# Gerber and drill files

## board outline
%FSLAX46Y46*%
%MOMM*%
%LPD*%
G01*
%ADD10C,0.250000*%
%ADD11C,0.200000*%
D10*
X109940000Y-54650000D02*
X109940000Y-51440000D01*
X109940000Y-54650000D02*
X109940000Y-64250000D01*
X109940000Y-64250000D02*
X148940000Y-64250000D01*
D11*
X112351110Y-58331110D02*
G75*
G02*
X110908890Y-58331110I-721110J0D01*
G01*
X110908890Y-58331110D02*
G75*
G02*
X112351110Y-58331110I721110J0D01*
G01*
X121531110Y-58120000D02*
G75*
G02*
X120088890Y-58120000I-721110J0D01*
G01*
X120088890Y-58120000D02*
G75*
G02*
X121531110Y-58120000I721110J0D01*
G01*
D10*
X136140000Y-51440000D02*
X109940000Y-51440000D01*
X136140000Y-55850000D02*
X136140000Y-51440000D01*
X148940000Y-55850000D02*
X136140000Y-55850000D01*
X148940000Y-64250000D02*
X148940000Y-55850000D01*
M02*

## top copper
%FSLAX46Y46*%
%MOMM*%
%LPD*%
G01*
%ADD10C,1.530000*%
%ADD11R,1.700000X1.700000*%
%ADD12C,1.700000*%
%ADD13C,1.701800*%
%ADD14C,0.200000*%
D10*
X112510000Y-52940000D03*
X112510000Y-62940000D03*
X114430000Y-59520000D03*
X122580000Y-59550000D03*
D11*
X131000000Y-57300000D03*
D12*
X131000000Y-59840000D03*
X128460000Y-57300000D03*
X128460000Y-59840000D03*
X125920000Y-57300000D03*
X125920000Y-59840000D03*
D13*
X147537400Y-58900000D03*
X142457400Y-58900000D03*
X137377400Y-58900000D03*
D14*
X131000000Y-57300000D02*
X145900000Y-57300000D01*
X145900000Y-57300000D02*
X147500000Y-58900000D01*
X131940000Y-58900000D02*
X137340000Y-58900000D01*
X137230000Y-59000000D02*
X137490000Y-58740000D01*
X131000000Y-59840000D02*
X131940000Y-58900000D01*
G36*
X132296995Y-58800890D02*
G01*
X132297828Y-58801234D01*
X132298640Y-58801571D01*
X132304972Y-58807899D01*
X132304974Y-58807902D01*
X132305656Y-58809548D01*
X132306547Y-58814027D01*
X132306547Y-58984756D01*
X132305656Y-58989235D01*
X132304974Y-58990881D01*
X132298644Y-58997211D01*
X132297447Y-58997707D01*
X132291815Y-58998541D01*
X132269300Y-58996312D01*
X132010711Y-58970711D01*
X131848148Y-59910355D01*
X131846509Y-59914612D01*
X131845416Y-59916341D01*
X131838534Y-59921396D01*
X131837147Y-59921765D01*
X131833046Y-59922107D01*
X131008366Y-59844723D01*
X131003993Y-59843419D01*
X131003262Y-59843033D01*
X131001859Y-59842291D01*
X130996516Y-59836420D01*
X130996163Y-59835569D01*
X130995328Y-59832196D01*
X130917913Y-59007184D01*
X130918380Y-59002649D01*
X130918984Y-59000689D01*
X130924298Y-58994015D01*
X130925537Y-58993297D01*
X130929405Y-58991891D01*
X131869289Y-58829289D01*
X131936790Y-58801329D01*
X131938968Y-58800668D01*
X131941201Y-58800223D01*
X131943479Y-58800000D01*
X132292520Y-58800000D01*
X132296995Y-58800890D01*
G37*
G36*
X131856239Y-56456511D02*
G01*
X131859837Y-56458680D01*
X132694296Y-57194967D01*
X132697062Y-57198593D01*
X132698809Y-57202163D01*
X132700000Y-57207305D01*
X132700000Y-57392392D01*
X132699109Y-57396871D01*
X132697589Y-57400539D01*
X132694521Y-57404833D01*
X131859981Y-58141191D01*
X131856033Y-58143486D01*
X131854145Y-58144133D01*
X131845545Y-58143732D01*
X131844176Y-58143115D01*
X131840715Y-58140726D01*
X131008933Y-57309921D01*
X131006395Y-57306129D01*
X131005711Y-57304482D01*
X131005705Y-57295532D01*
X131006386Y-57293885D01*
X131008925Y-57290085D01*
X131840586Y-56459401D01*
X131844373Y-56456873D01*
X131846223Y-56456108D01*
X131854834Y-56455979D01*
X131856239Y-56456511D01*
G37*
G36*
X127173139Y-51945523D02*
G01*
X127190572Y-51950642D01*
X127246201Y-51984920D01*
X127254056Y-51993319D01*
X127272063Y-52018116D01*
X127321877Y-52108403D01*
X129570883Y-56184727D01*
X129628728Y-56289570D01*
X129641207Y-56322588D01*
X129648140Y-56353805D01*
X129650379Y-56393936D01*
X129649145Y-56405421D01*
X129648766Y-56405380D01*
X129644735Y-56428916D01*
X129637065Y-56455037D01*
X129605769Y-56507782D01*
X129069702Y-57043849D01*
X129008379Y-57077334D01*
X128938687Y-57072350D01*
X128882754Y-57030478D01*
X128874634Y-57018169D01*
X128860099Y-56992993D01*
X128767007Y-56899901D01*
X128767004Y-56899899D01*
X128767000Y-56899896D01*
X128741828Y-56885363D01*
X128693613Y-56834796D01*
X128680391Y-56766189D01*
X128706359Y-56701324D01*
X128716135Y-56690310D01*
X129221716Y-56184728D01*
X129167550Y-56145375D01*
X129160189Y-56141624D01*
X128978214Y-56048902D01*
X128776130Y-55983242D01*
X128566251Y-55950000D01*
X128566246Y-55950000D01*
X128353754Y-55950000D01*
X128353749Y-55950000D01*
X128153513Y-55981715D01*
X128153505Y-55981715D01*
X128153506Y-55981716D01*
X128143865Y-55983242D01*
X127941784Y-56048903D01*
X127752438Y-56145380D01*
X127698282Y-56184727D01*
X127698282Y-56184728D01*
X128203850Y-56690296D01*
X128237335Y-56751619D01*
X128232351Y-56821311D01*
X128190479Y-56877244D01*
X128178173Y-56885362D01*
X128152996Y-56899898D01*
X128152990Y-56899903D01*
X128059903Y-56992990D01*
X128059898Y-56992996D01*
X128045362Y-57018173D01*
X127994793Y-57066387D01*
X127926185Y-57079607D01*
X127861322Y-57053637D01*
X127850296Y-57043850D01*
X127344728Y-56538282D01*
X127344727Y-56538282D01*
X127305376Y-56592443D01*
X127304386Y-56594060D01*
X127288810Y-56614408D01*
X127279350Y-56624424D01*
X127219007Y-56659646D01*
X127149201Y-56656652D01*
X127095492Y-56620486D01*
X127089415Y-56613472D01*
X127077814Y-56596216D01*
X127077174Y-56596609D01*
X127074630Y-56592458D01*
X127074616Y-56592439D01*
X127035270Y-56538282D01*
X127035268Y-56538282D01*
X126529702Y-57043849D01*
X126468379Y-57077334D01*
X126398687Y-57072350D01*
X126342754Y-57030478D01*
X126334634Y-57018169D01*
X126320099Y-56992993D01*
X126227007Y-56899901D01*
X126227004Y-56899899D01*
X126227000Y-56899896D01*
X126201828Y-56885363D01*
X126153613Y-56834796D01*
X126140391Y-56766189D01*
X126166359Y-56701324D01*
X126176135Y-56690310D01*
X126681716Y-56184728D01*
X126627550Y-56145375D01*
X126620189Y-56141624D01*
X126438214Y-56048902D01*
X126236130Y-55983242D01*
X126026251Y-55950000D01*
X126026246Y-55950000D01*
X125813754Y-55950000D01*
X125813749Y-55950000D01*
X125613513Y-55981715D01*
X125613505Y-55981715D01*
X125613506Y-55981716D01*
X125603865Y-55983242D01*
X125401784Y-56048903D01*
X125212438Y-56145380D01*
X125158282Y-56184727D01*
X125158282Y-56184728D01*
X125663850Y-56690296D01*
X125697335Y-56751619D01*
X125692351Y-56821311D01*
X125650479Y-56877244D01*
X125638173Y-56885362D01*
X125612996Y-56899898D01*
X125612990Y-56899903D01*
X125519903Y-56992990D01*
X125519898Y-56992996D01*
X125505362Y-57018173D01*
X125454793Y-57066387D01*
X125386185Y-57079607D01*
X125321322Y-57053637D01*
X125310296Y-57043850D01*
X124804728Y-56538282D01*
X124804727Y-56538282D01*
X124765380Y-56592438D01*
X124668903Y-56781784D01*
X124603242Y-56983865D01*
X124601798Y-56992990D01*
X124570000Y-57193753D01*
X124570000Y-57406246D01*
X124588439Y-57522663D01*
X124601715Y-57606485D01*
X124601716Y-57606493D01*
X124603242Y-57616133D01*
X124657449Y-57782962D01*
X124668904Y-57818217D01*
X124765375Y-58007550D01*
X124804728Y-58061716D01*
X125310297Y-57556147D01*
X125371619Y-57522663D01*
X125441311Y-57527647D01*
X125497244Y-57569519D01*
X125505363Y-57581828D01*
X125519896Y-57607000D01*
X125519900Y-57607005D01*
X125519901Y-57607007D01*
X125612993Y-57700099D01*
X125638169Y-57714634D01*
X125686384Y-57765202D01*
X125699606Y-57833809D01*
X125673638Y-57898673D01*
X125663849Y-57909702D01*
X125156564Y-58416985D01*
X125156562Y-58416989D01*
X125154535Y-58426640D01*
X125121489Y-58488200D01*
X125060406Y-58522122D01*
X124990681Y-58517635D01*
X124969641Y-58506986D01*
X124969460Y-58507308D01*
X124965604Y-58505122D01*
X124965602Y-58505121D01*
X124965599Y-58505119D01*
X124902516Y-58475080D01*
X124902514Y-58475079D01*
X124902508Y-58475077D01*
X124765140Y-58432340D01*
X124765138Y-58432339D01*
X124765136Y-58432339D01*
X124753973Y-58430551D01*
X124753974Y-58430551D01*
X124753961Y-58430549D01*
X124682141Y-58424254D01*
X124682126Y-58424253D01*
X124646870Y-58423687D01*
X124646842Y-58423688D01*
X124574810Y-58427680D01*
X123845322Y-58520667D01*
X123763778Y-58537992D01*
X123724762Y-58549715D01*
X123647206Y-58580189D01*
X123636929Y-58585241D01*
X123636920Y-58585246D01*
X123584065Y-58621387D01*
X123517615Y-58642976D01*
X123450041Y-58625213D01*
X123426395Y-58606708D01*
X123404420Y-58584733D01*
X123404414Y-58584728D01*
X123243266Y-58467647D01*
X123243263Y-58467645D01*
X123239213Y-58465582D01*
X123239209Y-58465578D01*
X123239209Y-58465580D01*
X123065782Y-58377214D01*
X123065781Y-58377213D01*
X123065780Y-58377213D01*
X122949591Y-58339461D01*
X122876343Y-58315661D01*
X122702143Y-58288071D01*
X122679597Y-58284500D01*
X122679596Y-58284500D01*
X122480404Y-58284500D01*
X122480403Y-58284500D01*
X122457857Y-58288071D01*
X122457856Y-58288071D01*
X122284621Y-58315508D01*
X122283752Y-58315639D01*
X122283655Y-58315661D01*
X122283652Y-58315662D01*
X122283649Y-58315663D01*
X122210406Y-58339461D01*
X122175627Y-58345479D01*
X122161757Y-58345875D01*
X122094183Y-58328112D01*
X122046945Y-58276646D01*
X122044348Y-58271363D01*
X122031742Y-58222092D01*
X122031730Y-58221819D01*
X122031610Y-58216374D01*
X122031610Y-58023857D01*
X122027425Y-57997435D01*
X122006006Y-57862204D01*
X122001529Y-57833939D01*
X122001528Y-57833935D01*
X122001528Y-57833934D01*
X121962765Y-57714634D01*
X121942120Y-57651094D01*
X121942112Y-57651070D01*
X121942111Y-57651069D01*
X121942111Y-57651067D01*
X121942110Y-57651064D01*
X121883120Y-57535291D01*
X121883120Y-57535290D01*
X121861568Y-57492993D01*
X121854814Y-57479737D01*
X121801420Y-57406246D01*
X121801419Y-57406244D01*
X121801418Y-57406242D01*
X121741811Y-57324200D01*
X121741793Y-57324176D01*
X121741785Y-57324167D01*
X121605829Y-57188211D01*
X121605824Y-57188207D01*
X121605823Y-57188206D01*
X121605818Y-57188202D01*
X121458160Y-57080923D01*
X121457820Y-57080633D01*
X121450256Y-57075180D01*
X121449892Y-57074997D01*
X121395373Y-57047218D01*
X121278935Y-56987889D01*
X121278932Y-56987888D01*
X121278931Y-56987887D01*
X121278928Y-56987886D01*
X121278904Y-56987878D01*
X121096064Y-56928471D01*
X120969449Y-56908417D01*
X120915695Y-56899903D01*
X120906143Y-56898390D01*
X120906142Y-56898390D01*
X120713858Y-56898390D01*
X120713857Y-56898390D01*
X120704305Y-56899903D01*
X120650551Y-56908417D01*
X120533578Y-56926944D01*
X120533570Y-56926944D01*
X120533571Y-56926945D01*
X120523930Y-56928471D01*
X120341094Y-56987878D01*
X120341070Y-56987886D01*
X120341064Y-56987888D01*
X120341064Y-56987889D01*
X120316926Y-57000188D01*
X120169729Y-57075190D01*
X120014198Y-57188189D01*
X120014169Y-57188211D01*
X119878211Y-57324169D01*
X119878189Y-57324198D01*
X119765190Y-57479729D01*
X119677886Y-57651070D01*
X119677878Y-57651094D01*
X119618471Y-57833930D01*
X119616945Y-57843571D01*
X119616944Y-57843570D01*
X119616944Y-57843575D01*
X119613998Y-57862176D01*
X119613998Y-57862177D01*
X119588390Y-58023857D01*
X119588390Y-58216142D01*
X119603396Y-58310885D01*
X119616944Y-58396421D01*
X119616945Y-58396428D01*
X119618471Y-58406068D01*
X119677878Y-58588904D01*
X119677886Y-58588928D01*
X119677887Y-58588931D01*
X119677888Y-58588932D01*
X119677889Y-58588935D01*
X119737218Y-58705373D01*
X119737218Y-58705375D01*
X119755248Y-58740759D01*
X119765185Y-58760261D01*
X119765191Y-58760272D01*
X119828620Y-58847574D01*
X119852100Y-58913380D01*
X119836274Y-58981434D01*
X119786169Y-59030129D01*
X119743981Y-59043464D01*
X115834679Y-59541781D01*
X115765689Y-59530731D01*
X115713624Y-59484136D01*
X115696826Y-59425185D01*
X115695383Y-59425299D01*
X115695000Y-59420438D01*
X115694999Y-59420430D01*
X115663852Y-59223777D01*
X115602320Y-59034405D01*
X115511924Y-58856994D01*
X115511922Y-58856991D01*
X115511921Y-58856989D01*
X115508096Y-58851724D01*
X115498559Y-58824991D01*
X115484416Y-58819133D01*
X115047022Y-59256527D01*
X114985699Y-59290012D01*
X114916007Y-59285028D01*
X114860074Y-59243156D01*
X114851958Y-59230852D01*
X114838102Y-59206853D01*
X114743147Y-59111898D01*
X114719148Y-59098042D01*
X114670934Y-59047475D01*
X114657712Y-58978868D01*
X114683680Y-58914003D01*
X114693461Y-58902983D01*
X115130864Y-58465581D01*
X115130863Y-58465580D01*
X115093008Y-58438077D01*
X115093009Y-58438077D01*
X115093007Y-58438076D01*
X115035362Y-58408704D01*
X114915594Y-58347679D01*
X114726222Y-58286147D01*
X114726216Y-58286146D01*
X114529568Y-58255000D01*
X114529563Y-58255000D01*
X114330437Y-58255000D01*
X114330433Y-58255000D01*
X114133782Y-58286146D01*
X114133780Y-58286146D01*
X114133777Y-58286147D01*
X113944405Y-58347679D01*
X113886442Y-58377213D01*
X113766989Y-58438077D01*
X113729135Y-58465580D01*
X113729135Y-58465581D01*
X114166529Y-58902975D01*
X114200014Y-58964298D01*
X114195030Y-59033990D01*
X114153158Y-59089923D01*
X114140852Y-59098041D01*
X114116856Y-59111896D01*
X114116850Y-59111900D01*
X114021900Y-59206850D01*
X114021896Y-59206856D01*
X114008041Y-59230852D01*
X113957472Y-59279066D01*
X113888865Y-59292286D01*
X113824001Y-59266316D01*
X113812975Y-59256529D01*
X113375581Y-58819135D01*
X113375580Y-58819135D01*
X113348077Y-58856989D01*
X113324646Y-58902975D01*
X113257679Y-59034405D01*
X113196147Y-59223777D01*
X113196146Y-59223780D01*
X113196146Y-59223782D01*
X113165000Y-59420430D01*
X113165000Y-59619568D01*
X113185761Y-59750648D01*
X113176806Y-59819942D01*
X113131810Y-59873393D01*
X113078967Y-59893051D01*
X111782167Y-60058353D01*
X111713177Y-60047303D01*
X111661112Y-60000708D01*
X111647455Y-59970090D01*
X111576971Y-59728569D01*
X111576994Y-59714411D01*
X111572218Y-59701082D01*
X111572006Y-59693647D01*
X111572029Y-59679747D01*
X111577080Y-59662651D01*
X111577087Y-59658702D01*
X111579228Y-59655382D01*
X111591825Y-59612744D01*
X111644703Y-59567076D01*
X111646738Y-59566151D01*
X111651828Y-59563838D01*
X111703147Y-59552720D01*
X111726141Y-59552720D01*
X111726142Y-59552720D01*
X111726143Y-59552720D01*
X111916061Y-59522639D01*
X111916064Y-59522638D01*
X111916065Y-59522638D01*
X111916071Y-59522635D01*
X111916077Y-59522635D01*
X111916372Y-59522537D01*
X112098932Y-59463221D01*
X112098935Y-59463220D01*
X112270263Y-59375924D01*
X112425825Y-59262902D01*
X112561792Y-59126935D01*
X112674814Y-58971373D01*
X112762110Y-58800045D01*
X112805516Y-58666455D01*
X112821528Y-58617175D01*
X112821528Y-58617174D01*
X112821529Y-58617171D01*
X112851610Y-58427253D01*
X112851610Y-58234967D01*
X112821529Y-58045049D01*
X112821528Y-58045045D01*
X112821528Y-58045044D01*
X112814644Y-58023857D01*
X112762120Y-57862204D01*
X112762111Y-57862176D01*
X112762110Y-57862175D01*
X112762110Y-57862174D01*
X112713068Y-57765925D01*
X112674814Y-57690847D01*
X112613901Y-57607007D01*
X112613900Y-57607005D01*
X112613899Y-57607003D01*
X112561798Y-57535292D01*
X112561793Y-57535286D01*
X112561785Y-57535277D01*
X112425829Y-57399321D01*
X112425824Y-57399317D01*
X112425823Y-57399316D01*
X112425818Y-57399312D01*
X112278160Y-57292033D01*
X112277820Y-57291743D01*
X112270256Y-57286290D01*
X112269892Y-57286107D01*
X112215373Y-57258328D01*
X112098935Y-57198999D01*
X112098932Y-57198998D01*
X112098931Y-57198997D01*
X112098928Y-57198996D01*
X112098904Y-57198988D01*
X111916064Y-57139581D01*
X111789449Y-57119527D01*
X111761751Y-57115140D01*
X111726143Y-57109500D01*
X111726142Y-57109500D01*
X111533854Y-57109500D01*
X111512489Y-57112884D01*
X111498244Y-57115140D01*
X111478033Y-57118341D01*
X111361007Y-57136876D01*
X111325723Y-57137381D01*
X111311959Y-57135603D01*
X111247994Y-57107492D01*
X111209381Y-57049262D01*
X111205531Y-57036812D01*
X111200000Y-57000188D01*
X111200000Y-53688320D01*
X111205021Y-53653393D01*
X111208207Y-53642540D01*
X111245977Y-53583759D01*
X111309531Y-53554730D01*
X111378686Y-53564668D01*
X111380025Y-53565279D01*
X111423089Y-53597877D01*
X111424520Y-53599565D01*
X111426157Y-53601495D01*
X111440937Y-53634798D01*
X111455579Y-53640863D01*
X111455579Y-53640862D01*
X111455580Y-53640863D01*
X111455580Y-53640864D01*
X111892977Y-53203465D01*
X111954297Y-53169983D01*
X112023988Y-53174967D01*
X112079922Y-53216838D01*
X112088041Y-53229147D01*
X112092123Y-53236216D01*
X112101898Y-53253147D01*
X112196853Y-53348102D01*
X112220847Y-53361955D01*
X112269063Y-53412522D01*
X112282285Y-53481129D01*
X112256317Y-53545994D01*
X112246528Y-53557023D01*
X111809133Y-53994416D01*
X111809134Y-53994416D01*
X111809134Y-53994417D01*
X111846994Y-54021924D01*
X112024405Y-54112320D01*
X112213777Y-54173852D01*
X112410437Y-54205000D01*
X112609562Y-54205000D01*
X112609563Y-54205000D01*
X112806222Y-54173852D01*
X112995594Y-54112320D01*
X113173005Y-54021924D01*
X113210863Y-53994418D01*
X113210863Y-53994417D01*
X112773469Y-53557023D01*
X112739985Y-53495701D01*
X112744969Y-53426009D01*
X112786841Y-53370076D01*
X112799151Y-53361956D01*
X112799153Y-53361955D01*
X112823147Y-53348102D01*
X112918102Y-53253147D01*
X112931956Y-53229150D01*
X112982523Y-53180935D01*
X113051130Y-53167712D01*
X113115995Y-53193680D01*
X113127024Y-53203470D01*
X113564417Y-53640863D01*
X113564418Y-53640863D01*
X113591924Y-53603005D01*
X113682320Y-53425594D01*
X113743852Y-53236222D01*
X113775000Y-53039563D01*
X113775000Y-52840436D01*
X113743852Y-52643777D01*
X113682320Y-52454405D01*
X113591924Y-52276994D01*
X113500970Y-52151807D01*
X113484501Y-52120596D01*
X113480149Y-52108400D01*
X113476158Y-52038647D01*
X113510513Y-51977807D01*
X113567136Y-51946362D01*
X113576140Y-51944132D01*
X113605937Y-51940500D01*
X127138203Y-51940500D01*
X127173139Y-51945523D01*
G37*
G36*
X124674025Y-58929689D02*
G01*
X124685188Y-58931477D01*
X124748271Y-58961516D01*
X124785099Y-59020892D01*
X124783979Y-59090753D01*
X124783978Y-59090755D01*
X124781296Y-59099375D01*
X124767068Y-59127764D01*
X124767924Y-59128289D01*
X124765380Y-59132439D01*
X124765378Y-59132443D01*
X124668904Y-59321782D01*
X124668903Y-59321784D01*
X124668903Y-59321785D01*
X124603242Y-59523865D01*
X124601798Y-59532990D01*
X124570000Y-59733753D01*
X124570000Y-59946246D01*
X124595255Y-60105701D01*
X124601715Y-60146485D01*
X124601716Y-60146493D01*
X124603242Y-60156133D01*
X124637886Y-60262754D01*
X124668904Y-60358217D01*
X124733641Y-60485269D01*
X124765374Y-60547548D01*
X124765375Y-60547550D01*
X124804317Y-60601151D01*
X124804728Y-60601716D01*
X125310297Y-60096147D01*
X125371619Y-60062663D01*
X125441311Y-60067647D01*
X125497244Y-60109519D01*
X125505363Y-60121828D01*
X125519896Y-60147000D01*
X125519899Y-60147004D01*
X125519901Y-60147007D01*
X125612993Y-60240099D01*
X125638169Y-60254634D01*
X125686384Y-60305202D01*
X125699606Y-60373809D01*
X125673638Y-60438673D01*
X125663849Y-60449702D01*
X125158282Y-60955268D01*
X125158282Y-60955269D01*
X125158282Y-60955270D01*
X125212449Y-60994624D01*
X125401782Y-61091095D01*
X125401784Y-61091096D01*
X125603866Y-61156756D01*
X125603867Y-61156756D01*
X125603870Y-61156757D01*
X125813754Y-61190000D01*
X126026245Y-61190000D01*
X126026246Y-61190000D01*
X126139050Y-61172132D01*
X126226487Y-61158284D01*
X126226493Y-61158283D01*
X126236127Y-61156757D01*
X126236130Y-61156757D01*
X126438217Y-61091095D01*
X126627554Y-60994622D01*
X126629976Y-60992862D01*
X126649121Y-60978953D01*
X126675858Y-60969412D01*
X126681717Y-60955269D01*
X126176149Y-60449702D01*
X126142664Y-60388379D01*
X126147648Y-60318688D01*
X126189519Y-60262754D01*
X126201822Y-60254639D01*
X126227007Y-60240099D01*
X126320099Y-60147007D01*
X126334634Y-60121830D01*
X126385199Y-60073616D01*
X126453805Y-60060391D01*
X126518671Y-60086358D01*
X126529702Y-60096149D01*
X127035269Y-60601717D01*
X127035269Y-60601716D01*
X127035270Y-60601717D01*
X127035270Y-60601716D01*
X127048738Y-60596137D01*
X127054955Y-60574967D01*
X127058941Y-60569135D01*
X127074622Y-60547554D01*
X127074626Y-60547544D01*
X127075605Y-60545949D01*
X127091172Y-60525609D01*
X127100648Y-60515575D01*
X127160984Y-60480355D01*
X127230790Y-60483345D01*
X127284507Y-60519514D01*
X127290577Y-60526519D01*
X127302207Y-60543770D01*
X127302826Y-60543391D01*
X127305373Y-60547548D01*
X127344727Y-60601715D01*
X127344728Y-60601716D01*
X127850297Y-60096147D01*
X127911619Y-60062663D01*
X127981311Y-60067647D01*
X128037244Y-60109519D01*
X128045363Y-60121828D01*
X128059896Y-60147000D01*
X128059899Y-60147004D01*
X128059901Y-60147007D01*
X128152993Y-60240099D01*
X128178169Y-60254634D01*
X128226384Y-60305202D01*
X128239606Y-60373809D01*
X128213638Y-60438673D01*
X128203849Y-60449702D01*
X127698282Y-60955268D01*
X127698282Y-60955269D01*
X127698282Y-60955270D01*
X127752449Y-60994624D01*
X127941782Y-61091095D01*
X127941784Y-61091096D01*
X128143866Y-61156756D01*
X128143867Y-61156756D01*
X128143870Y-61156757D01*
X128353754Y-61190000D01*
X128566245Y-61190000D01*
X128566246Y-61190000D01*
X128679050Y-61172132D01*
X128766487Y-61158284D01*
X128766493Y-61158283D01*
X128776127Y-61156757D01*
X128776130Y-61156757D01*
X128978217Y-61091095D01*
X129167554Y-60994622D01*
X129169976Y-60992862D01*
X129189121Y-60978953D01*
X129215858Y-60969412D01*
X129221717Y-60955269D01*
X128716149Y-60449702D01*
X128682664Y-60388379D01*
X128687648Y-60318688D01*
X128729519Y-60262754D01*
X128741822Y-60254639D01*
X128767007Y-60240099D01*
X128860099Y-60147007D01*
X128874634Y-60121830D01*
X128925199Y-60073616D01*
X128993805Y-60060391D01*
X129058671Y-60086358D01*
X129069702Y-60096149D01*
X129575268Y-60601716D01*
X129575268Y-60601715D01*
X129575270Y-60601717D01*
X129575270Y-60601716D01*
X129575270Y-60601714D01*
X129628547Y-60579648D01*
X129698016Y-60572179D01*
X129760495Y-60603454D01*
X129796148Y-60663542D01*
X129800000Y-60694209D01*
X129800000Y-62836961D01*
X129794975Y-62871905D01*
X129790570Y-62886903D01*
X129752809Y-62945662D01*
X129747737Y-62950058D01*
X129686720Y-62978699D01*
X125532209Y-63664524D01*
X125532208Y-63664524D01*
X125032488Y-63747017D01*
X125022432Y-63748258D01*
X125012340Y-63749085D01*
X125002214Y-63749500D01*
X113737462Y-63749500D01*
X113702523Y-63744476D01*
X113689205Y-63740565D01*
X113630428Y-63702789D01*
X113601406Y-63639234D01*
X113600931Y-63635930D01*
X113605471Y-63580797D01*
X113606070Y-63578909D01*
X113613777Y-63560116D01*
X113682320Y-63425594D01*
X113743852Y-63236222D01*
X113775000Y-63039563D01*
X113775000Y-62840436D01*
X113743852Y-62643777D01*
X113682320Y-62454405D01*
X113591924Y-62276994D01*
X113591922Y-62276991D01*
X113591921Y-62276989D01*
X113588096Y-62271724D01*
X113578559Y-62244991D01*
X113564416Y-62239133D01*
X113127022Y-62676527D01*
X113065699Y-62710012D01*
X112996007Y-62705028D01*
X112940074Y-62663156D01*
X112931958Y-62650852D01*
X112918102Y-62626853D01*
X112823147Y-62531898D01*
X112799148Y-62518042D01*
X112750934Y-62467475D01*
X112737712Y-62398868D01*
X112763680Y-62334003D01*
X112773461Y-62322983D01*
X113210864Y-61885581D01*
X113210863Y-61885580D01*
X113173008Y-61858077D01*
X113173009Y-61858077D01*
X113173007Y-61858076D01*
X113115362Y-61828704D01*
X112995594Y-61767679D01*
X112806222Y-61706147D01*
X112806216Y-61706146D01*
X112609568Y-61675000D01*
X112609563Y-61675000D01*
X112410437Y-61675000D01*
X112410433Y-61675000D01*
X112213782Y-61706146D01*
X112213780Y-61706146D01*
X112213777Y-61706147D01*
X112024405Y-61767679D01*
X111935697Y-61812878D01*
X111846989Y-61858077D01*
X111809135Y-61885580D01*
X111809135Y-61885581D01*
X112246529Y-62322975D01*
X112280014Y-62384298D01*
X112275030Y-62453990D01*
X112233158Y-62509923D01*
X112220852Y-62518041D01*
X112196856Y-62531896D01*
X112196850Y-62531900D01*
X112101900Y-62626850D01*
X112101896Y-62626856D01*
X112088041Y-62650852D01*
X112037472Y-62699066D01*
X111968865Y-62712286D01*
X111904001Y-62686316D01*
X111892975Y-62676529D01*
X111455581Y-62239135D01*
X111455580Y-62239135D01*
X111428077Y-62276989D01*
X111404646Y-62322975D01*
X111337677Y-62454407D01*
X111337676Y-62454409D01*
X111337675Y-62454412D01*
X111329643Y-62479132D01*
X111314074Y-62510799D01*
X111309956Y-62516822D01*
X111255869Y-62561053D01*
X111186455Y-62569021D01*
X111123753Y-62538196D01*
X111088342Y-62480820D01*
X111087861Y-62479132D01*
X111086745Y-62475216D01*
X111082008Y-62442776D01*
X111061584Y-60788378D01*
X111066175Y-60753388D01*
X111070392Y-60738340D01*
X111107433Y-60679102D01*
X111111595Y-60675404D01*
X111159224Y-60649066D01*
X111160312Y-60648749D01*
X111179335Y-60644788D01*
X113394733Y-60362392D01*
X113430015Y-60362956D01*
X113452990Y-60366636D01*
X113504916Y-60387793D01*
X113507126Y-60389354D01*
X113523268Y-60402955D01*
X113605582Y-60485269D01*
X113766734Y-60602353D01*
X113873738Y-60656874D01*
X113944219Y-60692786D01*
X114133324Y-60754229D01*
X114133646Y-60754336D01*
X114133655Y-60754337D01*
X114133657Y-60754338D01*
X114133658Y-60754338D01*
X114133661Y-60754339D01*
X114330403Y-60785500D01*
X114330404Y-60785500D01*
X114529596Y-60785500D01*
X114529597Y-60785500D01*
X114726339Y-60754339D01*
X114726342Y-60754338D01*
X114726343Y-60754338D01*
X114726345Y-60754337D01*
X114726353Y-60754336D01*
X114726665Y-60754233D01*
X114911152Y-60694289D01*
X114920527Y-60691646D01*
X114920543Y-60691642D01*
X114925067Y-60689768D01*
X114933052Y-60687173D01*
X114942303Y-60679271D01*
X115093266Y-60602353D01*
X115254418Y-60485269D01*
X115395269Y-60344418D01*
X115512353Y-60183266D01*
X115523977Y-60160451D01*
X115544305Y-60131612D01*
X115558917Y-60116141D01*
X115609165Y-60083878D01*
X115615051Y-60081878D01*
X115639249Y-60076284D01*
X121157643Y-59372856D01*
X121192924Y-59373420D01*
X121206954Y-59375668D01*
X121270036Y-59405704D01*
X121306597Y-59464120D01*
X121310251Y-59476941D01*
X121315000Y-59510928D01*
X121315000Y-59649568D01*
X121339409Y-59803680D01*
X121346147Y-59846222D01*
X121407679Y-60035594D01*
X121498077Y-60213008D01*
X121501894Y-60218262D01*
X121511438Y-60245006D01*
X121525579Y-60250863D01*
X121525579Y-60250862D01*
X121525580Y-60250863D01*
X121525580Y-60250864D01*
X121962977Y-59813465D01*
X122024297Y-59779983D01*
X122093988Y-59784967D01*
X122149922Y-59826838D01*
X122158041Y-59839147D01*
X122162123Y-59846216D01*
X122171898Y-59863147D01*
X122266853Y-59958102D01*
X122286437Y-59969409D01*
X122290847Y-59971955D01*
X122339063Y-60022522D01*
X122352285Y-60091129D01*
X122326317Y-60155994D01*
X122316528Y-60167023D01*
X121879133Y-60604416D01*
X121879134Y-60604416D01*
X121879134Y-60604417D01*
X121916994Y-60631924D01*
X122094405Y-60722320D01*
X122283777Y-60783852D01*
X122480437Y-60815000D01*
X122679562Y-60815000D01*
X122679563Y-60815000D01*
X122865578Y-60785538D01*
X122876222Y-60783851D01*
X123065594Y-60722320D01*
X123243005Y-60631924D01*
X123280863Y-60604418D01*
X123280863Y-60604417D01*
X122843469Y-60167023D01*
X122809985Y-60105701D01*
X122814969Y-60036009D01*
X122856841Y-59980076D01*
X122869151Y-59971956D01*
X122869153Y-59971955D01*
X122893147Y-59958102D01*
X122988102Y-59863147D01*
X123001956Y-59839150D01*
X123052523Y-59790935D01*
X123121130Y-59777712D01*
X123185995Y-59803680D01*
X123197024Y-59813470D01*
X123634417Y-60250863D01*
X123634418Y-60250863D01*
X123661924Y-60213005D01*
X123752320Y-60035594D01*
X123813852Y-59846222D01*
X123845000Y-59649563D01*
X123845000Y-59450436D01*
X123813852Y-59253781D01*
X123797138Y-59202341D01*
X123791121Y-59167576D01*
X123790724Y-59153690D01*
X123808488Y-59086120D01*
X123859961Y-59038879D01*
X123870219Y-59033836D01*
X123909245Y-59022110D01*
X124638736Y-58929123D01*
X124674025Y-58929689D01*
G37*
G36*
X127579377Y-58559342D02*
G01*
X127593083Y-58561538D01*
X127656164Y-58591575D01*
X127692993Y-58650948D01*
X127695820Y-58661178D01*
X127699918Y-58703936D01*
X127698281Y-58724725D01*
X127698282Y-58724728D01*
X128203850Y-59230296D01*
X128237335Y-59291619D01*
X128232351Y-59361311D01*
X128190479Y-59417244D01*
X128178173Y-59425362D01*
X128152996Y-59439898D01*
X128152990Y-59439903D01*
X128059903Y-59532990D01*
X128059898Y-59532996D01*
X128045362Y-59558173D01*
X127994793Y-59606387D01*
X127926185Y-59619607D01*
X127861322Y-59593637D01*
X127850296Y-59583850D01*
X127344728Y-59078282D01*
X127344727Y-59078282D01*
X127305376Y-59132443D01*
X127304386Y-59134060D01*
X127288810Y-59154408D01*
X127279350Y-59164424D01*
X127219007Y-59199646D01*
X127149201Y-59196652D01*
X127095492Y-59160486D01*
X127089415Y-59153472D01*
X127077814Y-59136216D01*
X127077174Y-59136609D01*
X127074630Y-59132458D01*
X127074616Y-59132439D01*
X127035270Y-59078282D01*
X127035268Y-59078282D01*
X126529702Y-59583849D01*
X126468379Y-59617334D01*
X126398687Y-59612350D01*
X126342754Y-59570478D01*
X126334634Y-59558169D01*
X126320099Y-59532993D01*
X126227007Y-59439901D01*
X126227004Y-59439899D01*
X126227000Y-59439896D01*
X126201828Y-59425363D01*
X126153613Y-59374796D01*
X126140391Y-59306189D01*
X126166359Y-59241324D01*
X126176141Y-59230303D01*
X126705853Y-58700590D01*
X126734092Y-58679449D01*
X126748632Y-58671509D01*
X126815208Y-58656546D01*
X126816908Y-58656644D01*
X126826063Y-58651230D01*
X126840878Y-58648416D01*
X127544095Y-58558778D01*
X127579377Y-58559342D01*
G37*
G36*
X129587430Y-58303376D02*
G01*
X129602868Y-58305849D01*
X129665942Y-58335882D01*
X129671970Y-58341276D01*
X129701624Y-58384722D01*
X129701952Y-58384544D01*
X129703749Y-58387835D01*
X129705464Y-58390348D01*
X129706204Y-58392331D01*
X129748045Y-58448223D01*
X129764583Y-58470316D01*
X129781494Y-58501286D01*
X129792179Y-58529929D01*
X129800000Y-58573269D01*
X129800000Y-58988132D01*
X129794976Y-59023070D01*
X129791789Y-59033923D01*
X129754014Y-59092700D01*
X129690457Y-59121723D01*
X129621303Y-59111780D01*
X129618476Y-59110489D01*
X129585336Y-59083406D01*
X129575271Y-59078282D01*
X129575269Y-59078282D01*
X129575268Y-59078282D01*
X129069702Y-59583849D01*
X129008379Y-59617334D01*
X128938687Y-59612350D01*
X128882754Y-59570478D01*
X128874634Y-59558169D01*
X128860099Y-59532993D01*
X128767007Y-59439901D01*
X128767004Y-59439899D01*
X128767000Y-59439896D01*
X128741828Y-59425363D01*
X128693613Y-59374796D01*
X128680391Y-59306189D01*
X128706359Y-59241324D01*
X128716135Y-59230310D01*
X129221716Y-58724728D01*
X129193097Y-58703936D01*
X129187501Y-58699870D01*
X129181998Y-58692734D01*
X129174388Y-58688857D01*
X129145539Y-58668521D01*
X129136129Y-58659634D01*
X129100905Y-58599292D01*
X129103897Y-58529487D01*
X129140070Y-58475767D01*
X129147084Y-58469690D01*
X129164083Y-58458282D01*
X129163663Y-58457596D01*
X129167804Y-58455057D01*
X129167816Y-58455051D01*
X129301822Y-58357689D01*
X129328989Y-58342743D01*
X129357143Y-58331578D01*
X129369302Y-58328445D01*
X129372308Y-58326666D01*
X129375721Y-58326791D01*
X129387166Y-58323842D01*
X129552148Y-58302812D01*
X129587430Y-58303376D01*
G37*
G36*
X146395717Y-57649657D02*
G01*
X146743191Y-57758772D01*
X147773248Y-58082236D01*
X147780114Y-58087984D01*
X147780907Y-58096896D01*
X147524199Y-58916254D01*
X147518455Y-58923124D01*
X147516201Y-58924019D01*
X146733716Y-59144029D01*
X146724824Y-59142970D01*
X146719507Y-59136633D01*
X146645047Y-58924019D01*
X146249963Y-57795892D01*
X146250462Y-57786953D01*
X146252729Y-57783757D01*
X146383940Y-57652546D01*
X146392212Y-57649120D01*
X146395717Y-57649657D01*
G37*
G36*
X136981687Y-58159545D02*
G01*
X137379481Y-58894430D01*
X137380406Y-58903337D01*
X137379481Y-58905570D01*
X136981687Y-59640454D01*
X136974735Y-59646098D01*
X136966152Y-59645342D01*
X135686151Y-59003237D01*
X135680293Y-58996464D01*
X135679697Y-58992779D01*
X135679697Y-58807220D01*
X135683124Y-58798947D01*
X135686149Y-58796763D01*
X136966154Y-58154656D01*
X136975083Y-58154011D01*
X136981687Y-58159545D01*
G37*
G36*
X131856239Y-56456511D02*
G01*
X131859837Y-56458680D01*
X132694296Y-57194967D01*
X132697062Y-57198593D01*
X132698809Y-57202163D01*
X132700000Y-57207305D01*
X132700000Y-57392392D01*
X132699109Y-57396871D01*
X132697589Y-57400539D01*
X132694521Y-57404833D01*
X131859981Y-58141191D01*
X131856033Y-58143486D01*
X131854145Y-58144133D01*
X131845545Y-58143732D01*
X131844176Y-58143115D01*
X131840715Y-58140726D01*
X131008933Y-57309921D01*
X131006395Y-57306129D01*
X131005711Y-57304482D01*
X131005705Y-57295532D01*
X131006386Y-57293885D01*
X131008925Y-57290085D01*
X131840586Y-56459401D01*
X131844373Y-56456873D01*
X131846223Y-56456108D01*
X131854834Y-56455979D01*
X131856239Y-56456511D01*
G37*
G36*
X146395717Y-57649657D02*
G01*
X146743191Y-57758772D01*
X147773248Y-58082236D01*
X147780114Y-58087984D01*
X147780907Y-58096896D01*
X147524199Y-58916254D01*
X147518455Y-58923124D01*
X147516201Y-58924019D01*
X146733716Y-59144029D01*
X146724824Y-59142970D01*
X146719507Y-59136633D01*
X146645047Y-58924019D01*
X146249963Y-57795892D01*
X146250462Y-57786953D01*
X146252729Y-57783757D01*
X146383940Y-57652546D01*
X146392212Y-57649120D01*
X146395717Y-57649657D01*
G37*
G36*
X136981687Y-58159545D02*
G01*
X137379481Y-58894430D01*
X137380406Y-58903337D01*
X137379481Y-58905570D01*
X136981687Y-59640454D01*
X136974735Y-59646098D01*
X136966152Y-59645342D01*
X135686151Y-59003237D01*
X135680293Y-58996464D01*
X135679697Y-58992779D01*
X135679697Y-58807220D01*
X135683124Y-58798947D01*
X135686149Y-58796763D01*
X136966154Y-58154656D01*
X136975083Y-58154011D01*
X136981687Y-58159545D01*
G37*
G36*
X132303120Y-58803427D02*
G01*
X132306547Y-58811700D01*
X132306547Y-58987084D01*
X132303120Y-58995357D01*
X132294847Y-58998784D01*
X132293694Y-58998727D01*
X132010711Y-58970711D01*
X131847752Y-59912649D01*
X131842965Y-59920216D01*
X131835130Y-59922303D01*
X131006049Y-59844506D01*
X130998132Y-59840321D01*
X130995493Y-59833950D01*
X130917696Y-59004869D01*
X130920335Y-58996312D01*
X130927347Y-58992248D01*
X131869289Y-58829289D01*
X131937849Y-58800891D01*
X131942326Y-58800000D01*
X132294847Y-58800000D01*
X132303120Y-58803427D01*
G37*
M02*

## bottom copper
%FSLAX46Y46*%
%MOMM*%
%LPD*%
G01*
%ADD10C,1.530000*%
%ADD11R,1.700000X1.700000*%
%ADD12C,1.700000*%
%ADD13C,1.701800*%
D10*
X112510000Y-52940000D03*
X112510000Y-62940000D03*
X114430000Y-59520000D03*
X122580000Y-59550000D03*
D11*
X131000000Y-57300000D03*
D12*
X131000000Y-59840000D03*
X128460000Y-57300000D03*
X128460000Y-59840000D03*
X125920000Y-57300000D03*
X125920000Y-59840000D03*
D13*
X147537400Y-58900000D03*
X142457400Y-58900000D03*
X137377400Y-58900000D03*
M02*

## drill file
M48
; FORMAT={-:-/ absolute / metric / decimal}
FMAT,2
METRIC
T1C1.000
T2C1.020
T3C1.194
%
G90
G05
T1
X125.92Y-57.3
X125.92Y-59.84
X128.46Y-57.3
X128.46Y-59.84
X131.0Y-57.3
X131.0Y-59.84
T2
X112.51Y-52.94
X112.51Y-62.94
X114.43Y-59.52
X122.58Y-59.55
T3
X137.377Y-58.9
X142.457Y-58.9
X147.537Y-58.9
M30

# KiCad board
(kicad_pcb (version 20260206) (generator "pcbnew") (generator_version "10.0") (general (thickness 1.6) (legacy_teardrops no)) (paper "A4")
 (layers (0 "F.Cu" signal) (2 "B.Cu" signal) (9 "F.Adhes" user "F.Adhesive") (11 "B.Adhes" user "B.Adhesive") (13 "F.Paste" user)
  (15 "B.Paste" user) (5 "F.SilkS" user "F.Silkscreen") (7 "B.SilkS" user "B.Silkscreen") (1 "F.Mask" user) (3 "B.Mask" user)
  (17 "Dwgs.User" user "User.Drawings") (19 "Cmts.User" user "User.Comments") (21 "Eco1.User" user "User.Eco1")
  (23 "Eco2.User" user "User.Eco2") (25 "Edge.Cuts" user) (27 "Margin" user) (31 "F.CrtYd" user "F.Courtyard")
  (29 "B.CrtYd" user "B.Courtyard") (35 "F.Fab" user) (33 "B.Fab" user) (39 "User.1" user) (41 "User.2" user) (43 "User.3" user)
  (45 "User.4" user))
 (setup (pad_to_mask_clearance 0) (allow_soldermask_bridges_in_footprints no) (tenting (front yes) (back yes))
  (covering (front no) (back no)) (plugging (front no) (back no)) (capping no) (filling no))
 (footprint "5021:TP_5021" (layer "F.Cu") (at 112.51 52.94 -90)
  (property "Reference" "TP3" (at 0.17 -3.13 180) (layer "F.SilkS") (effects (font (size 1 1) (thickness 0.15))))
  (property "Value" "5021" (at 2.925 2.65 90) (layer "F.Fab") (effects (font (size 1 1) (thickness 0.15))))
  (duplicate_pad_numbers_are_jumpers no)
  (pad "TP" thru_hole circle (at 0 0 270) (size 1.53 1.53) (drill 1.02) (layers "*.Cu" "*.Mask") (remove_unused_layers no)
   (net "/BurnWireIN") (solder_mask_margin 0.102)
   (teardrops (best_length_ratio 0.5) (max_length 1) (best_width_ratio 1) (max_width 2) (curved_edges no) (filter_ratio 0.9) (enabled yes)
    (allow_two_segments yes) (prefer_zone_connections yes))))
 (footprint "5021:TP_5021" (layer "F.Cu") (at 112.51 62.94 -90)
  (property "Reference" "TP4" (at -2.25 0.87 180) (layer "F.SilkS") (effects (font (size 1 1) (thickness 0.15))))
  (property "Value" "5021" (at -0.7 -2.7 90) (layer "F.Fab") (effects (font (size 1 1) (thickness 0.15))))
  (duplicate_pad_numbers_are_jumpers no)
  (pad "TP" thru_hole circle (at 0 0 270) (size 1.53 1.53) (drill 1.02) (layers "*.Cu" "*.Mask") (remove_unused_layers no) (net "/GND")
   (solder_mask_margin 0.102)
   (teardrops (best_length_ratio 0.5) (max_length 1) (best_width_ratio 1) (max_width 2) (curved_edges no) (filter_ratio 0.9) (enabled yes)
    (allow_two_segments yes) (prefer_zone_connections yes))))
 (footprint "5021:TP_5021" (layer "F.Cu") (at 114.43 59.52)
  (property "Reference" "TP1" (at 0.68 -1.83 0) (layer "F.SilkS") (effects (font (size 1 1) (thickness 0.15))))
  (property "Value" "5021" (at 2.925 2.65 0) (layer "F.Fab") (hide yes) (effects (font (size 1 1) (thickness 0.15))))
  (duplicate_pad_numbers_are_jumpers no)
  (pad "TP" thru_hole circle (at 0 0) (size 1.53 1.53) (drill 1.02) (layers "*.Cu" "*.Mask") (remove_unused_layers no) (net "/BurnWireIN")
   (solder_mask_margin 0.102)
   (teardrops (best_length_ratio 0.5) (max_length 1) (best_width_ratio 1) (max_width 2) (curved_edges no) (filter_ratio 0.9) (enabled yes)
    (allow_two_segments yes) (prefer_zone_connections yes))))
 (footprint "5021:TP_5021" (layer "F.Cu") (at 122.58 59.55)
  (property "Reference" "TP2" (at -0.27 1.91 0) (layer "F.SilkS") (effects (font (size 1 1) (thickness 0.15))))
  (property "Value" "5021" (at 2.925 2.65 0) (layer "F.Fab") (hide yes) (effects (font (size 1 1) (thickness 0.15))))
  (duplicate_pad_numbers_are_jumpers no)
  (pad "TP" thru_hole circle (at 0 0) (size 1.53 1.53) (drill 1.02) (layers "*.Cu" "*.Mask") (remove_unused_layers no) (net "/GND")
   (solder_mask_margin 0.102)
   (teardrops (best_length_ratio 0.5) (max_length 1) (best_width_ratio 1) (max_width 2) (curved_edges no) (filter_ratio 0.9) (enabled yes)
    (allow_two_segments yes) (prefer_zone_connections yes))))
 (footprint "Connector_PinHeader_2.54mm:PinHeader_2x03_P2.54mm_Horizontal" (layer "F.Cu") (at 131 57.3 -90)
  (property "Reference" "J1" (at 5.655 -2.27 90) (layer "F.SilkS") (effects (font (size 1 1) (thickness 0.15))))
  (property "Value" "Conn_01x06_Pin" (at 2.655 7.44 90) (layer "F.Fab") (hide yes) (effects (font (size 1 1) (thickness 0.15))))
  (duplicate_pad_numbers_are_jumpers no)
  (pad "1" thru_hole rect (at 0 0 270) (size 1.7 1.7) (drill 1) (layers "*.Cu" "*.Mask") (remove_unused_layers no)
   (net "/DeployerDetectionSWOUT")
   (teardrops (best_length_ratio 0.5) (max_length 1) (best_width_ratio 1) (max_width 2) (curved_edges no) (filter_ratio 0.9) (enabled yes)
    (allow_two_segments yes) (prefer_zone_connections yes)))
  (pad "2" thru_hole circle (at 2.54 0 270) (size 1.7 1.7) (drill 1) (layers "*.Cu" "*.Mask") (remove_unused_layers no)
   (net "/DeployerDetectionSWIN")
   (teardrops (best_length_ratio 0.5) (max_length 1) (best_width_ratio 1) (max_width 2) (curved_edges no) (filter_ratio 0.9) (enabled yes)
    (allow_two_segments yes) (prefer_zone_connections yes)))
  (pad "3" thru_hole circle (at 0 2.54 270) (size 1.7 1.7) (drill 1) (layers "*.Cu" "*.Mask") (remove_unused_layers no) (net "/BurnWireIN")
   (teardrops (best_length_ratio 0.5) (max_length 1) (best_width_ratio 1) (max_width 2) (curved_edges no) (filter_ratio 0.9) (enabled yes)
    (allow_two_segments yes) (prefer_zone_connections yes)))
  (pad "4" thru_hole circle (at 2.54 2.54 270) (size 1.7 1.7) (drill 1) (layers "*.Cu" "*.Mask") (remove_unused_layers no) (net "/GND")
   (teardrops (best_length_ratio 0.5) (max_length 1) (best_width_ratio 1) (max_width 2) (curved_edges no) (filter_ratio 0.9) (enabled yes)
    (allow_two_segments yes) (prefer_zone_connections yes)))
  (pad "5" thru_hole circle (at 0 5.08 270) (size 1.7 1.7) (drill 1) (layers "*.Cu" "*.Mask") (remove_unused_layers no) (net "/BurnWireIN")
   (teardrops (best_length_ratio 0.5) (max_length 1) (best_width_ratio 1) (max_width 2) (curved_edges no) (filter_ratio 0.9) (enabled yes)
    (allow_two_segments yes) (prefer_zone_connections yes)))
  (pad "6" thru_hole circle (at 2.54 5.08 270) (size 1.7 1.7) (drill 1) (layers "*.Cu" "*.Mask") (remove_unused_layers no) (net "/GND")
   (teardrops (best_length_ratio 0.5) (max_length 1) (best_width_ratio 1) (max_width 2) (curved_edges no) (filter_ratio 0.9) (enabled yes)
    (allow_two_segments yes) (prefer_zone_connections yes))))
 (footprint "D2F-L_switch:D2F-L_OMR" (layer "B.Cu") (at 147.5374 58.9 180)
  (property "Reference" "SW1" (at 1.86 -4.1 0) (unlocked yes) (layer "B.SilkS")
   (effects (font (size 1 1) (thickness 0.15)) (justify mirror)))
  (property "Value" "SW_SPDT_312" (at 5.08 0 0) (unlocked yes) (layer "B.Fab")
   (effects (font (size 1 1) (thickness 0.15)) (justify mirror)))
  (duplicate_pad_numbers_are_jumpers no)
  (pad "1" thru_hole circle (at 0 0 180) (size 1.7018 1.7018) (drill 1.1938) (layers "*.Cu" "*.Mask") (remove_unused_layers no)
   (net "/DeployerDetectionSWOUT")
   (teardrops (best_length_ratio 0.5) (max_length 1) (best_width_ratio 1) (max_width 2) (curved_edges no) (filter_ratio 0.9) (enabled yes)
    (allow_two_segments yes) (prefer_zone_connections yes)))
  (pad "2" thru_hole circle (at 5.08 0 180) (size 1.7018 1.7018) (drill 1.1938) (layers "*.Cu" "*.Mask") (remove_unused_layers no)
   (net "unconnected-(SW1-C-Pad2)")
   (teardrops (best_length_ratio 0.5) (max_length 1) (best_width_ratio 1) (max_width 2) (curved_edges no) (filter_ratio 0.9) (enabled yes)
    (allow_two_segments yes) (prefer_zone_connections yes)))
  (pad "3" thru_hole circle (at 10.16 0 180) (size 1.7018 1.7018) (drill 1.1938) (layers "*.Cu" "*.Mask") (remove_unused_layers no)
   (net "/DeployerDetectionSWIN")
   (teardrops (best_length_ratio 0.5) (max_length 1) (best_width_ratio 1) (max_width 2) (curved_edges no) (filter_ratio 0.9) (enabled yes)
    (allow_two_segments yes) (prefer_zone_connections yes))))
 (gr_line (start 109.94 54.65) (end 109.94 51.44) (stroke (width 0.25) (type solid)) (layer "Edge.Cuts"))
 (gr_line (start 109.94 54.65) (end 109.94 64.25) (stroke (width 0.25) (type default)) (layer "Edge.Cuts"))
 (gr_line (start 109.94 64.25) (end 148.94 64.25) (stroke (width 0.25) (type solid)) (layer "Edge.Cuts"))
 (gr_circle (center 111.63 58.33111) (end 112.23 58.73111) (stroke (width 0.2) (type solid)) (fill no) (layer "Edge.Cuts"))
 (gr_circle (center 120.81 58.12) (end 121.41 58.52) (stroke (width 0.2) (type solid)) (fill no) (layer "Edge.Cuts"))
 (gr_line (start 136.14 51.44) (end 109.94 51.44) (stroke (width 0.25) (type default)) (layer "Edge.Cuts"))
 (gr_line (start 136.14 55.85) (end 136.14 51.44) (stroke (width 0.25) (type solid)) (layer "Edge.Cuts"))
 (gr_line (start 148.94 55.85) (end 136.14 55.85) (stroke (width 0.25) (type default)) (layer "Edge.Cuts"))
 (gr_line (start 148.94 64.25) (end 148.94 55.85) (stroke (width 0.25) (type default)) (layer "Edge.Cuts"))
 (segment (start 131 57.3) (end 145.9 57.3) (width 0.2) (layer "F.Cu") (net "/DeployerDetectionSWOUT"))
 (segment (start 145.9 57.3) (end 147.5 58.9) (width 0.2) (layer "F.Cu") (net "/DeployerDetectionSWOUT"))
 (segment (start 131.94 58.9) (end 137.34 58.9) (width 0.2) (layer "F.Cu") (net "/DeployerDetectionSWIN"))
 (segment (start 137.23 59) (end 137.49 58.74) (width 0.2) (layer "F.Cu") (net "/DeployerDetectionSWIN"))
 (segment (start 131 59.84) (end 131.94 58.9) (width 0.2) (layer "F.Cu") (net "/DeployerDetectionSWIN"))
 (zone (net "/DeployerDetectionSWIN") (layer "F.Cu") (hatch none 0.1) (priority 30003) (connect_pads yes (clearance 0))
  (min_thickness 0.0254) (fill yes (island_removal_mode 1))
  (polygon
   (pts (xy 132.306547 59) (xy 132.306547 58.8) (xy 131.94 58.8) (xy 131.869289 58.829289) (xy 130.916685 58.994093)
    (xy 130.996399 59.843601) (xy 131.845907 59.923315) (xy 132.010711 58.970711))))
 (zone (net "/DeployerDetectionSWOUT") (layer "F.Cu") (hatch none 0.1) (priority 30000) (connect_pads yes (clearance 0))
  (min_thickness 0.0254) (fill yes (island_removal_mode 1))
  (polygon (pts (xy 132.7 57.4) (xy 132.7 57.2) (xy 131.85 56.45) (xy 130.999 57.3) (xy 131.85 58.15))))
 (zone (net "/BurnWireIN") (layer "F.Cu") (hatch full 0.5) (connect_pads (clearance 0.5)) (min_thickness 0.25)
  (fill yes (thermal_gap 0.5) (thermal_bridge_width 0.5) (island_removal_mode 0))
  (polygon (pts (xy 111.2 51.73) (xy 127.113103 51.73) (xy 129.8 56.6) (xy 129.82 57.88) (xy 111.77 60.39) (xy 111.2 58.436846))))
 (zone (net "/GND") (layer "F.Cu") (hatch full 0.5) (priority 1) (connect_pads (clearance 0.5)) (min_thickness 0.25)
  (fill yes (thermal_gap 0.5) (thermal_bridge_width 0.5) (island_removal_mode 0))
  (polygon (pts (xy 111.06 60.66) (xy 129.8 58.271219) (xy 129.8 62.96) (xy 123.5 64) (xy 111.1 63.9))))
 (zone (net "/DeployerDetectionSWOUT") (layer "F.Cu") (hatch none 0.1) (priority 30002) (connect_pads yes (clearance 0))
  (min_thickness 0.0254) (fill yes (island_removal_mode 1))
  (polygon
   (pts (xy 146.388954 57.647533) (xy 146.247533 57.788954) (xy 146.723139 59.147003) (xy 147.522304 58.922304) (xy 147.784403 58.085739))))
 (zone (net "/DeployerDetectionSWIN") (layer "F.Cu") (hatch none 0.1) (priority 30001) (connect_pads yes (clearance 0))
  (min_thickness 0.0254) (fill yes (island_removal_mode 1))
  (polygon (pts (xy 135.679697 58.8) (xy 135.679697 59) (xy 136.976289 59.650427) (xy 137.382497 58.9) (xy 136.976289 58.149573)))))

